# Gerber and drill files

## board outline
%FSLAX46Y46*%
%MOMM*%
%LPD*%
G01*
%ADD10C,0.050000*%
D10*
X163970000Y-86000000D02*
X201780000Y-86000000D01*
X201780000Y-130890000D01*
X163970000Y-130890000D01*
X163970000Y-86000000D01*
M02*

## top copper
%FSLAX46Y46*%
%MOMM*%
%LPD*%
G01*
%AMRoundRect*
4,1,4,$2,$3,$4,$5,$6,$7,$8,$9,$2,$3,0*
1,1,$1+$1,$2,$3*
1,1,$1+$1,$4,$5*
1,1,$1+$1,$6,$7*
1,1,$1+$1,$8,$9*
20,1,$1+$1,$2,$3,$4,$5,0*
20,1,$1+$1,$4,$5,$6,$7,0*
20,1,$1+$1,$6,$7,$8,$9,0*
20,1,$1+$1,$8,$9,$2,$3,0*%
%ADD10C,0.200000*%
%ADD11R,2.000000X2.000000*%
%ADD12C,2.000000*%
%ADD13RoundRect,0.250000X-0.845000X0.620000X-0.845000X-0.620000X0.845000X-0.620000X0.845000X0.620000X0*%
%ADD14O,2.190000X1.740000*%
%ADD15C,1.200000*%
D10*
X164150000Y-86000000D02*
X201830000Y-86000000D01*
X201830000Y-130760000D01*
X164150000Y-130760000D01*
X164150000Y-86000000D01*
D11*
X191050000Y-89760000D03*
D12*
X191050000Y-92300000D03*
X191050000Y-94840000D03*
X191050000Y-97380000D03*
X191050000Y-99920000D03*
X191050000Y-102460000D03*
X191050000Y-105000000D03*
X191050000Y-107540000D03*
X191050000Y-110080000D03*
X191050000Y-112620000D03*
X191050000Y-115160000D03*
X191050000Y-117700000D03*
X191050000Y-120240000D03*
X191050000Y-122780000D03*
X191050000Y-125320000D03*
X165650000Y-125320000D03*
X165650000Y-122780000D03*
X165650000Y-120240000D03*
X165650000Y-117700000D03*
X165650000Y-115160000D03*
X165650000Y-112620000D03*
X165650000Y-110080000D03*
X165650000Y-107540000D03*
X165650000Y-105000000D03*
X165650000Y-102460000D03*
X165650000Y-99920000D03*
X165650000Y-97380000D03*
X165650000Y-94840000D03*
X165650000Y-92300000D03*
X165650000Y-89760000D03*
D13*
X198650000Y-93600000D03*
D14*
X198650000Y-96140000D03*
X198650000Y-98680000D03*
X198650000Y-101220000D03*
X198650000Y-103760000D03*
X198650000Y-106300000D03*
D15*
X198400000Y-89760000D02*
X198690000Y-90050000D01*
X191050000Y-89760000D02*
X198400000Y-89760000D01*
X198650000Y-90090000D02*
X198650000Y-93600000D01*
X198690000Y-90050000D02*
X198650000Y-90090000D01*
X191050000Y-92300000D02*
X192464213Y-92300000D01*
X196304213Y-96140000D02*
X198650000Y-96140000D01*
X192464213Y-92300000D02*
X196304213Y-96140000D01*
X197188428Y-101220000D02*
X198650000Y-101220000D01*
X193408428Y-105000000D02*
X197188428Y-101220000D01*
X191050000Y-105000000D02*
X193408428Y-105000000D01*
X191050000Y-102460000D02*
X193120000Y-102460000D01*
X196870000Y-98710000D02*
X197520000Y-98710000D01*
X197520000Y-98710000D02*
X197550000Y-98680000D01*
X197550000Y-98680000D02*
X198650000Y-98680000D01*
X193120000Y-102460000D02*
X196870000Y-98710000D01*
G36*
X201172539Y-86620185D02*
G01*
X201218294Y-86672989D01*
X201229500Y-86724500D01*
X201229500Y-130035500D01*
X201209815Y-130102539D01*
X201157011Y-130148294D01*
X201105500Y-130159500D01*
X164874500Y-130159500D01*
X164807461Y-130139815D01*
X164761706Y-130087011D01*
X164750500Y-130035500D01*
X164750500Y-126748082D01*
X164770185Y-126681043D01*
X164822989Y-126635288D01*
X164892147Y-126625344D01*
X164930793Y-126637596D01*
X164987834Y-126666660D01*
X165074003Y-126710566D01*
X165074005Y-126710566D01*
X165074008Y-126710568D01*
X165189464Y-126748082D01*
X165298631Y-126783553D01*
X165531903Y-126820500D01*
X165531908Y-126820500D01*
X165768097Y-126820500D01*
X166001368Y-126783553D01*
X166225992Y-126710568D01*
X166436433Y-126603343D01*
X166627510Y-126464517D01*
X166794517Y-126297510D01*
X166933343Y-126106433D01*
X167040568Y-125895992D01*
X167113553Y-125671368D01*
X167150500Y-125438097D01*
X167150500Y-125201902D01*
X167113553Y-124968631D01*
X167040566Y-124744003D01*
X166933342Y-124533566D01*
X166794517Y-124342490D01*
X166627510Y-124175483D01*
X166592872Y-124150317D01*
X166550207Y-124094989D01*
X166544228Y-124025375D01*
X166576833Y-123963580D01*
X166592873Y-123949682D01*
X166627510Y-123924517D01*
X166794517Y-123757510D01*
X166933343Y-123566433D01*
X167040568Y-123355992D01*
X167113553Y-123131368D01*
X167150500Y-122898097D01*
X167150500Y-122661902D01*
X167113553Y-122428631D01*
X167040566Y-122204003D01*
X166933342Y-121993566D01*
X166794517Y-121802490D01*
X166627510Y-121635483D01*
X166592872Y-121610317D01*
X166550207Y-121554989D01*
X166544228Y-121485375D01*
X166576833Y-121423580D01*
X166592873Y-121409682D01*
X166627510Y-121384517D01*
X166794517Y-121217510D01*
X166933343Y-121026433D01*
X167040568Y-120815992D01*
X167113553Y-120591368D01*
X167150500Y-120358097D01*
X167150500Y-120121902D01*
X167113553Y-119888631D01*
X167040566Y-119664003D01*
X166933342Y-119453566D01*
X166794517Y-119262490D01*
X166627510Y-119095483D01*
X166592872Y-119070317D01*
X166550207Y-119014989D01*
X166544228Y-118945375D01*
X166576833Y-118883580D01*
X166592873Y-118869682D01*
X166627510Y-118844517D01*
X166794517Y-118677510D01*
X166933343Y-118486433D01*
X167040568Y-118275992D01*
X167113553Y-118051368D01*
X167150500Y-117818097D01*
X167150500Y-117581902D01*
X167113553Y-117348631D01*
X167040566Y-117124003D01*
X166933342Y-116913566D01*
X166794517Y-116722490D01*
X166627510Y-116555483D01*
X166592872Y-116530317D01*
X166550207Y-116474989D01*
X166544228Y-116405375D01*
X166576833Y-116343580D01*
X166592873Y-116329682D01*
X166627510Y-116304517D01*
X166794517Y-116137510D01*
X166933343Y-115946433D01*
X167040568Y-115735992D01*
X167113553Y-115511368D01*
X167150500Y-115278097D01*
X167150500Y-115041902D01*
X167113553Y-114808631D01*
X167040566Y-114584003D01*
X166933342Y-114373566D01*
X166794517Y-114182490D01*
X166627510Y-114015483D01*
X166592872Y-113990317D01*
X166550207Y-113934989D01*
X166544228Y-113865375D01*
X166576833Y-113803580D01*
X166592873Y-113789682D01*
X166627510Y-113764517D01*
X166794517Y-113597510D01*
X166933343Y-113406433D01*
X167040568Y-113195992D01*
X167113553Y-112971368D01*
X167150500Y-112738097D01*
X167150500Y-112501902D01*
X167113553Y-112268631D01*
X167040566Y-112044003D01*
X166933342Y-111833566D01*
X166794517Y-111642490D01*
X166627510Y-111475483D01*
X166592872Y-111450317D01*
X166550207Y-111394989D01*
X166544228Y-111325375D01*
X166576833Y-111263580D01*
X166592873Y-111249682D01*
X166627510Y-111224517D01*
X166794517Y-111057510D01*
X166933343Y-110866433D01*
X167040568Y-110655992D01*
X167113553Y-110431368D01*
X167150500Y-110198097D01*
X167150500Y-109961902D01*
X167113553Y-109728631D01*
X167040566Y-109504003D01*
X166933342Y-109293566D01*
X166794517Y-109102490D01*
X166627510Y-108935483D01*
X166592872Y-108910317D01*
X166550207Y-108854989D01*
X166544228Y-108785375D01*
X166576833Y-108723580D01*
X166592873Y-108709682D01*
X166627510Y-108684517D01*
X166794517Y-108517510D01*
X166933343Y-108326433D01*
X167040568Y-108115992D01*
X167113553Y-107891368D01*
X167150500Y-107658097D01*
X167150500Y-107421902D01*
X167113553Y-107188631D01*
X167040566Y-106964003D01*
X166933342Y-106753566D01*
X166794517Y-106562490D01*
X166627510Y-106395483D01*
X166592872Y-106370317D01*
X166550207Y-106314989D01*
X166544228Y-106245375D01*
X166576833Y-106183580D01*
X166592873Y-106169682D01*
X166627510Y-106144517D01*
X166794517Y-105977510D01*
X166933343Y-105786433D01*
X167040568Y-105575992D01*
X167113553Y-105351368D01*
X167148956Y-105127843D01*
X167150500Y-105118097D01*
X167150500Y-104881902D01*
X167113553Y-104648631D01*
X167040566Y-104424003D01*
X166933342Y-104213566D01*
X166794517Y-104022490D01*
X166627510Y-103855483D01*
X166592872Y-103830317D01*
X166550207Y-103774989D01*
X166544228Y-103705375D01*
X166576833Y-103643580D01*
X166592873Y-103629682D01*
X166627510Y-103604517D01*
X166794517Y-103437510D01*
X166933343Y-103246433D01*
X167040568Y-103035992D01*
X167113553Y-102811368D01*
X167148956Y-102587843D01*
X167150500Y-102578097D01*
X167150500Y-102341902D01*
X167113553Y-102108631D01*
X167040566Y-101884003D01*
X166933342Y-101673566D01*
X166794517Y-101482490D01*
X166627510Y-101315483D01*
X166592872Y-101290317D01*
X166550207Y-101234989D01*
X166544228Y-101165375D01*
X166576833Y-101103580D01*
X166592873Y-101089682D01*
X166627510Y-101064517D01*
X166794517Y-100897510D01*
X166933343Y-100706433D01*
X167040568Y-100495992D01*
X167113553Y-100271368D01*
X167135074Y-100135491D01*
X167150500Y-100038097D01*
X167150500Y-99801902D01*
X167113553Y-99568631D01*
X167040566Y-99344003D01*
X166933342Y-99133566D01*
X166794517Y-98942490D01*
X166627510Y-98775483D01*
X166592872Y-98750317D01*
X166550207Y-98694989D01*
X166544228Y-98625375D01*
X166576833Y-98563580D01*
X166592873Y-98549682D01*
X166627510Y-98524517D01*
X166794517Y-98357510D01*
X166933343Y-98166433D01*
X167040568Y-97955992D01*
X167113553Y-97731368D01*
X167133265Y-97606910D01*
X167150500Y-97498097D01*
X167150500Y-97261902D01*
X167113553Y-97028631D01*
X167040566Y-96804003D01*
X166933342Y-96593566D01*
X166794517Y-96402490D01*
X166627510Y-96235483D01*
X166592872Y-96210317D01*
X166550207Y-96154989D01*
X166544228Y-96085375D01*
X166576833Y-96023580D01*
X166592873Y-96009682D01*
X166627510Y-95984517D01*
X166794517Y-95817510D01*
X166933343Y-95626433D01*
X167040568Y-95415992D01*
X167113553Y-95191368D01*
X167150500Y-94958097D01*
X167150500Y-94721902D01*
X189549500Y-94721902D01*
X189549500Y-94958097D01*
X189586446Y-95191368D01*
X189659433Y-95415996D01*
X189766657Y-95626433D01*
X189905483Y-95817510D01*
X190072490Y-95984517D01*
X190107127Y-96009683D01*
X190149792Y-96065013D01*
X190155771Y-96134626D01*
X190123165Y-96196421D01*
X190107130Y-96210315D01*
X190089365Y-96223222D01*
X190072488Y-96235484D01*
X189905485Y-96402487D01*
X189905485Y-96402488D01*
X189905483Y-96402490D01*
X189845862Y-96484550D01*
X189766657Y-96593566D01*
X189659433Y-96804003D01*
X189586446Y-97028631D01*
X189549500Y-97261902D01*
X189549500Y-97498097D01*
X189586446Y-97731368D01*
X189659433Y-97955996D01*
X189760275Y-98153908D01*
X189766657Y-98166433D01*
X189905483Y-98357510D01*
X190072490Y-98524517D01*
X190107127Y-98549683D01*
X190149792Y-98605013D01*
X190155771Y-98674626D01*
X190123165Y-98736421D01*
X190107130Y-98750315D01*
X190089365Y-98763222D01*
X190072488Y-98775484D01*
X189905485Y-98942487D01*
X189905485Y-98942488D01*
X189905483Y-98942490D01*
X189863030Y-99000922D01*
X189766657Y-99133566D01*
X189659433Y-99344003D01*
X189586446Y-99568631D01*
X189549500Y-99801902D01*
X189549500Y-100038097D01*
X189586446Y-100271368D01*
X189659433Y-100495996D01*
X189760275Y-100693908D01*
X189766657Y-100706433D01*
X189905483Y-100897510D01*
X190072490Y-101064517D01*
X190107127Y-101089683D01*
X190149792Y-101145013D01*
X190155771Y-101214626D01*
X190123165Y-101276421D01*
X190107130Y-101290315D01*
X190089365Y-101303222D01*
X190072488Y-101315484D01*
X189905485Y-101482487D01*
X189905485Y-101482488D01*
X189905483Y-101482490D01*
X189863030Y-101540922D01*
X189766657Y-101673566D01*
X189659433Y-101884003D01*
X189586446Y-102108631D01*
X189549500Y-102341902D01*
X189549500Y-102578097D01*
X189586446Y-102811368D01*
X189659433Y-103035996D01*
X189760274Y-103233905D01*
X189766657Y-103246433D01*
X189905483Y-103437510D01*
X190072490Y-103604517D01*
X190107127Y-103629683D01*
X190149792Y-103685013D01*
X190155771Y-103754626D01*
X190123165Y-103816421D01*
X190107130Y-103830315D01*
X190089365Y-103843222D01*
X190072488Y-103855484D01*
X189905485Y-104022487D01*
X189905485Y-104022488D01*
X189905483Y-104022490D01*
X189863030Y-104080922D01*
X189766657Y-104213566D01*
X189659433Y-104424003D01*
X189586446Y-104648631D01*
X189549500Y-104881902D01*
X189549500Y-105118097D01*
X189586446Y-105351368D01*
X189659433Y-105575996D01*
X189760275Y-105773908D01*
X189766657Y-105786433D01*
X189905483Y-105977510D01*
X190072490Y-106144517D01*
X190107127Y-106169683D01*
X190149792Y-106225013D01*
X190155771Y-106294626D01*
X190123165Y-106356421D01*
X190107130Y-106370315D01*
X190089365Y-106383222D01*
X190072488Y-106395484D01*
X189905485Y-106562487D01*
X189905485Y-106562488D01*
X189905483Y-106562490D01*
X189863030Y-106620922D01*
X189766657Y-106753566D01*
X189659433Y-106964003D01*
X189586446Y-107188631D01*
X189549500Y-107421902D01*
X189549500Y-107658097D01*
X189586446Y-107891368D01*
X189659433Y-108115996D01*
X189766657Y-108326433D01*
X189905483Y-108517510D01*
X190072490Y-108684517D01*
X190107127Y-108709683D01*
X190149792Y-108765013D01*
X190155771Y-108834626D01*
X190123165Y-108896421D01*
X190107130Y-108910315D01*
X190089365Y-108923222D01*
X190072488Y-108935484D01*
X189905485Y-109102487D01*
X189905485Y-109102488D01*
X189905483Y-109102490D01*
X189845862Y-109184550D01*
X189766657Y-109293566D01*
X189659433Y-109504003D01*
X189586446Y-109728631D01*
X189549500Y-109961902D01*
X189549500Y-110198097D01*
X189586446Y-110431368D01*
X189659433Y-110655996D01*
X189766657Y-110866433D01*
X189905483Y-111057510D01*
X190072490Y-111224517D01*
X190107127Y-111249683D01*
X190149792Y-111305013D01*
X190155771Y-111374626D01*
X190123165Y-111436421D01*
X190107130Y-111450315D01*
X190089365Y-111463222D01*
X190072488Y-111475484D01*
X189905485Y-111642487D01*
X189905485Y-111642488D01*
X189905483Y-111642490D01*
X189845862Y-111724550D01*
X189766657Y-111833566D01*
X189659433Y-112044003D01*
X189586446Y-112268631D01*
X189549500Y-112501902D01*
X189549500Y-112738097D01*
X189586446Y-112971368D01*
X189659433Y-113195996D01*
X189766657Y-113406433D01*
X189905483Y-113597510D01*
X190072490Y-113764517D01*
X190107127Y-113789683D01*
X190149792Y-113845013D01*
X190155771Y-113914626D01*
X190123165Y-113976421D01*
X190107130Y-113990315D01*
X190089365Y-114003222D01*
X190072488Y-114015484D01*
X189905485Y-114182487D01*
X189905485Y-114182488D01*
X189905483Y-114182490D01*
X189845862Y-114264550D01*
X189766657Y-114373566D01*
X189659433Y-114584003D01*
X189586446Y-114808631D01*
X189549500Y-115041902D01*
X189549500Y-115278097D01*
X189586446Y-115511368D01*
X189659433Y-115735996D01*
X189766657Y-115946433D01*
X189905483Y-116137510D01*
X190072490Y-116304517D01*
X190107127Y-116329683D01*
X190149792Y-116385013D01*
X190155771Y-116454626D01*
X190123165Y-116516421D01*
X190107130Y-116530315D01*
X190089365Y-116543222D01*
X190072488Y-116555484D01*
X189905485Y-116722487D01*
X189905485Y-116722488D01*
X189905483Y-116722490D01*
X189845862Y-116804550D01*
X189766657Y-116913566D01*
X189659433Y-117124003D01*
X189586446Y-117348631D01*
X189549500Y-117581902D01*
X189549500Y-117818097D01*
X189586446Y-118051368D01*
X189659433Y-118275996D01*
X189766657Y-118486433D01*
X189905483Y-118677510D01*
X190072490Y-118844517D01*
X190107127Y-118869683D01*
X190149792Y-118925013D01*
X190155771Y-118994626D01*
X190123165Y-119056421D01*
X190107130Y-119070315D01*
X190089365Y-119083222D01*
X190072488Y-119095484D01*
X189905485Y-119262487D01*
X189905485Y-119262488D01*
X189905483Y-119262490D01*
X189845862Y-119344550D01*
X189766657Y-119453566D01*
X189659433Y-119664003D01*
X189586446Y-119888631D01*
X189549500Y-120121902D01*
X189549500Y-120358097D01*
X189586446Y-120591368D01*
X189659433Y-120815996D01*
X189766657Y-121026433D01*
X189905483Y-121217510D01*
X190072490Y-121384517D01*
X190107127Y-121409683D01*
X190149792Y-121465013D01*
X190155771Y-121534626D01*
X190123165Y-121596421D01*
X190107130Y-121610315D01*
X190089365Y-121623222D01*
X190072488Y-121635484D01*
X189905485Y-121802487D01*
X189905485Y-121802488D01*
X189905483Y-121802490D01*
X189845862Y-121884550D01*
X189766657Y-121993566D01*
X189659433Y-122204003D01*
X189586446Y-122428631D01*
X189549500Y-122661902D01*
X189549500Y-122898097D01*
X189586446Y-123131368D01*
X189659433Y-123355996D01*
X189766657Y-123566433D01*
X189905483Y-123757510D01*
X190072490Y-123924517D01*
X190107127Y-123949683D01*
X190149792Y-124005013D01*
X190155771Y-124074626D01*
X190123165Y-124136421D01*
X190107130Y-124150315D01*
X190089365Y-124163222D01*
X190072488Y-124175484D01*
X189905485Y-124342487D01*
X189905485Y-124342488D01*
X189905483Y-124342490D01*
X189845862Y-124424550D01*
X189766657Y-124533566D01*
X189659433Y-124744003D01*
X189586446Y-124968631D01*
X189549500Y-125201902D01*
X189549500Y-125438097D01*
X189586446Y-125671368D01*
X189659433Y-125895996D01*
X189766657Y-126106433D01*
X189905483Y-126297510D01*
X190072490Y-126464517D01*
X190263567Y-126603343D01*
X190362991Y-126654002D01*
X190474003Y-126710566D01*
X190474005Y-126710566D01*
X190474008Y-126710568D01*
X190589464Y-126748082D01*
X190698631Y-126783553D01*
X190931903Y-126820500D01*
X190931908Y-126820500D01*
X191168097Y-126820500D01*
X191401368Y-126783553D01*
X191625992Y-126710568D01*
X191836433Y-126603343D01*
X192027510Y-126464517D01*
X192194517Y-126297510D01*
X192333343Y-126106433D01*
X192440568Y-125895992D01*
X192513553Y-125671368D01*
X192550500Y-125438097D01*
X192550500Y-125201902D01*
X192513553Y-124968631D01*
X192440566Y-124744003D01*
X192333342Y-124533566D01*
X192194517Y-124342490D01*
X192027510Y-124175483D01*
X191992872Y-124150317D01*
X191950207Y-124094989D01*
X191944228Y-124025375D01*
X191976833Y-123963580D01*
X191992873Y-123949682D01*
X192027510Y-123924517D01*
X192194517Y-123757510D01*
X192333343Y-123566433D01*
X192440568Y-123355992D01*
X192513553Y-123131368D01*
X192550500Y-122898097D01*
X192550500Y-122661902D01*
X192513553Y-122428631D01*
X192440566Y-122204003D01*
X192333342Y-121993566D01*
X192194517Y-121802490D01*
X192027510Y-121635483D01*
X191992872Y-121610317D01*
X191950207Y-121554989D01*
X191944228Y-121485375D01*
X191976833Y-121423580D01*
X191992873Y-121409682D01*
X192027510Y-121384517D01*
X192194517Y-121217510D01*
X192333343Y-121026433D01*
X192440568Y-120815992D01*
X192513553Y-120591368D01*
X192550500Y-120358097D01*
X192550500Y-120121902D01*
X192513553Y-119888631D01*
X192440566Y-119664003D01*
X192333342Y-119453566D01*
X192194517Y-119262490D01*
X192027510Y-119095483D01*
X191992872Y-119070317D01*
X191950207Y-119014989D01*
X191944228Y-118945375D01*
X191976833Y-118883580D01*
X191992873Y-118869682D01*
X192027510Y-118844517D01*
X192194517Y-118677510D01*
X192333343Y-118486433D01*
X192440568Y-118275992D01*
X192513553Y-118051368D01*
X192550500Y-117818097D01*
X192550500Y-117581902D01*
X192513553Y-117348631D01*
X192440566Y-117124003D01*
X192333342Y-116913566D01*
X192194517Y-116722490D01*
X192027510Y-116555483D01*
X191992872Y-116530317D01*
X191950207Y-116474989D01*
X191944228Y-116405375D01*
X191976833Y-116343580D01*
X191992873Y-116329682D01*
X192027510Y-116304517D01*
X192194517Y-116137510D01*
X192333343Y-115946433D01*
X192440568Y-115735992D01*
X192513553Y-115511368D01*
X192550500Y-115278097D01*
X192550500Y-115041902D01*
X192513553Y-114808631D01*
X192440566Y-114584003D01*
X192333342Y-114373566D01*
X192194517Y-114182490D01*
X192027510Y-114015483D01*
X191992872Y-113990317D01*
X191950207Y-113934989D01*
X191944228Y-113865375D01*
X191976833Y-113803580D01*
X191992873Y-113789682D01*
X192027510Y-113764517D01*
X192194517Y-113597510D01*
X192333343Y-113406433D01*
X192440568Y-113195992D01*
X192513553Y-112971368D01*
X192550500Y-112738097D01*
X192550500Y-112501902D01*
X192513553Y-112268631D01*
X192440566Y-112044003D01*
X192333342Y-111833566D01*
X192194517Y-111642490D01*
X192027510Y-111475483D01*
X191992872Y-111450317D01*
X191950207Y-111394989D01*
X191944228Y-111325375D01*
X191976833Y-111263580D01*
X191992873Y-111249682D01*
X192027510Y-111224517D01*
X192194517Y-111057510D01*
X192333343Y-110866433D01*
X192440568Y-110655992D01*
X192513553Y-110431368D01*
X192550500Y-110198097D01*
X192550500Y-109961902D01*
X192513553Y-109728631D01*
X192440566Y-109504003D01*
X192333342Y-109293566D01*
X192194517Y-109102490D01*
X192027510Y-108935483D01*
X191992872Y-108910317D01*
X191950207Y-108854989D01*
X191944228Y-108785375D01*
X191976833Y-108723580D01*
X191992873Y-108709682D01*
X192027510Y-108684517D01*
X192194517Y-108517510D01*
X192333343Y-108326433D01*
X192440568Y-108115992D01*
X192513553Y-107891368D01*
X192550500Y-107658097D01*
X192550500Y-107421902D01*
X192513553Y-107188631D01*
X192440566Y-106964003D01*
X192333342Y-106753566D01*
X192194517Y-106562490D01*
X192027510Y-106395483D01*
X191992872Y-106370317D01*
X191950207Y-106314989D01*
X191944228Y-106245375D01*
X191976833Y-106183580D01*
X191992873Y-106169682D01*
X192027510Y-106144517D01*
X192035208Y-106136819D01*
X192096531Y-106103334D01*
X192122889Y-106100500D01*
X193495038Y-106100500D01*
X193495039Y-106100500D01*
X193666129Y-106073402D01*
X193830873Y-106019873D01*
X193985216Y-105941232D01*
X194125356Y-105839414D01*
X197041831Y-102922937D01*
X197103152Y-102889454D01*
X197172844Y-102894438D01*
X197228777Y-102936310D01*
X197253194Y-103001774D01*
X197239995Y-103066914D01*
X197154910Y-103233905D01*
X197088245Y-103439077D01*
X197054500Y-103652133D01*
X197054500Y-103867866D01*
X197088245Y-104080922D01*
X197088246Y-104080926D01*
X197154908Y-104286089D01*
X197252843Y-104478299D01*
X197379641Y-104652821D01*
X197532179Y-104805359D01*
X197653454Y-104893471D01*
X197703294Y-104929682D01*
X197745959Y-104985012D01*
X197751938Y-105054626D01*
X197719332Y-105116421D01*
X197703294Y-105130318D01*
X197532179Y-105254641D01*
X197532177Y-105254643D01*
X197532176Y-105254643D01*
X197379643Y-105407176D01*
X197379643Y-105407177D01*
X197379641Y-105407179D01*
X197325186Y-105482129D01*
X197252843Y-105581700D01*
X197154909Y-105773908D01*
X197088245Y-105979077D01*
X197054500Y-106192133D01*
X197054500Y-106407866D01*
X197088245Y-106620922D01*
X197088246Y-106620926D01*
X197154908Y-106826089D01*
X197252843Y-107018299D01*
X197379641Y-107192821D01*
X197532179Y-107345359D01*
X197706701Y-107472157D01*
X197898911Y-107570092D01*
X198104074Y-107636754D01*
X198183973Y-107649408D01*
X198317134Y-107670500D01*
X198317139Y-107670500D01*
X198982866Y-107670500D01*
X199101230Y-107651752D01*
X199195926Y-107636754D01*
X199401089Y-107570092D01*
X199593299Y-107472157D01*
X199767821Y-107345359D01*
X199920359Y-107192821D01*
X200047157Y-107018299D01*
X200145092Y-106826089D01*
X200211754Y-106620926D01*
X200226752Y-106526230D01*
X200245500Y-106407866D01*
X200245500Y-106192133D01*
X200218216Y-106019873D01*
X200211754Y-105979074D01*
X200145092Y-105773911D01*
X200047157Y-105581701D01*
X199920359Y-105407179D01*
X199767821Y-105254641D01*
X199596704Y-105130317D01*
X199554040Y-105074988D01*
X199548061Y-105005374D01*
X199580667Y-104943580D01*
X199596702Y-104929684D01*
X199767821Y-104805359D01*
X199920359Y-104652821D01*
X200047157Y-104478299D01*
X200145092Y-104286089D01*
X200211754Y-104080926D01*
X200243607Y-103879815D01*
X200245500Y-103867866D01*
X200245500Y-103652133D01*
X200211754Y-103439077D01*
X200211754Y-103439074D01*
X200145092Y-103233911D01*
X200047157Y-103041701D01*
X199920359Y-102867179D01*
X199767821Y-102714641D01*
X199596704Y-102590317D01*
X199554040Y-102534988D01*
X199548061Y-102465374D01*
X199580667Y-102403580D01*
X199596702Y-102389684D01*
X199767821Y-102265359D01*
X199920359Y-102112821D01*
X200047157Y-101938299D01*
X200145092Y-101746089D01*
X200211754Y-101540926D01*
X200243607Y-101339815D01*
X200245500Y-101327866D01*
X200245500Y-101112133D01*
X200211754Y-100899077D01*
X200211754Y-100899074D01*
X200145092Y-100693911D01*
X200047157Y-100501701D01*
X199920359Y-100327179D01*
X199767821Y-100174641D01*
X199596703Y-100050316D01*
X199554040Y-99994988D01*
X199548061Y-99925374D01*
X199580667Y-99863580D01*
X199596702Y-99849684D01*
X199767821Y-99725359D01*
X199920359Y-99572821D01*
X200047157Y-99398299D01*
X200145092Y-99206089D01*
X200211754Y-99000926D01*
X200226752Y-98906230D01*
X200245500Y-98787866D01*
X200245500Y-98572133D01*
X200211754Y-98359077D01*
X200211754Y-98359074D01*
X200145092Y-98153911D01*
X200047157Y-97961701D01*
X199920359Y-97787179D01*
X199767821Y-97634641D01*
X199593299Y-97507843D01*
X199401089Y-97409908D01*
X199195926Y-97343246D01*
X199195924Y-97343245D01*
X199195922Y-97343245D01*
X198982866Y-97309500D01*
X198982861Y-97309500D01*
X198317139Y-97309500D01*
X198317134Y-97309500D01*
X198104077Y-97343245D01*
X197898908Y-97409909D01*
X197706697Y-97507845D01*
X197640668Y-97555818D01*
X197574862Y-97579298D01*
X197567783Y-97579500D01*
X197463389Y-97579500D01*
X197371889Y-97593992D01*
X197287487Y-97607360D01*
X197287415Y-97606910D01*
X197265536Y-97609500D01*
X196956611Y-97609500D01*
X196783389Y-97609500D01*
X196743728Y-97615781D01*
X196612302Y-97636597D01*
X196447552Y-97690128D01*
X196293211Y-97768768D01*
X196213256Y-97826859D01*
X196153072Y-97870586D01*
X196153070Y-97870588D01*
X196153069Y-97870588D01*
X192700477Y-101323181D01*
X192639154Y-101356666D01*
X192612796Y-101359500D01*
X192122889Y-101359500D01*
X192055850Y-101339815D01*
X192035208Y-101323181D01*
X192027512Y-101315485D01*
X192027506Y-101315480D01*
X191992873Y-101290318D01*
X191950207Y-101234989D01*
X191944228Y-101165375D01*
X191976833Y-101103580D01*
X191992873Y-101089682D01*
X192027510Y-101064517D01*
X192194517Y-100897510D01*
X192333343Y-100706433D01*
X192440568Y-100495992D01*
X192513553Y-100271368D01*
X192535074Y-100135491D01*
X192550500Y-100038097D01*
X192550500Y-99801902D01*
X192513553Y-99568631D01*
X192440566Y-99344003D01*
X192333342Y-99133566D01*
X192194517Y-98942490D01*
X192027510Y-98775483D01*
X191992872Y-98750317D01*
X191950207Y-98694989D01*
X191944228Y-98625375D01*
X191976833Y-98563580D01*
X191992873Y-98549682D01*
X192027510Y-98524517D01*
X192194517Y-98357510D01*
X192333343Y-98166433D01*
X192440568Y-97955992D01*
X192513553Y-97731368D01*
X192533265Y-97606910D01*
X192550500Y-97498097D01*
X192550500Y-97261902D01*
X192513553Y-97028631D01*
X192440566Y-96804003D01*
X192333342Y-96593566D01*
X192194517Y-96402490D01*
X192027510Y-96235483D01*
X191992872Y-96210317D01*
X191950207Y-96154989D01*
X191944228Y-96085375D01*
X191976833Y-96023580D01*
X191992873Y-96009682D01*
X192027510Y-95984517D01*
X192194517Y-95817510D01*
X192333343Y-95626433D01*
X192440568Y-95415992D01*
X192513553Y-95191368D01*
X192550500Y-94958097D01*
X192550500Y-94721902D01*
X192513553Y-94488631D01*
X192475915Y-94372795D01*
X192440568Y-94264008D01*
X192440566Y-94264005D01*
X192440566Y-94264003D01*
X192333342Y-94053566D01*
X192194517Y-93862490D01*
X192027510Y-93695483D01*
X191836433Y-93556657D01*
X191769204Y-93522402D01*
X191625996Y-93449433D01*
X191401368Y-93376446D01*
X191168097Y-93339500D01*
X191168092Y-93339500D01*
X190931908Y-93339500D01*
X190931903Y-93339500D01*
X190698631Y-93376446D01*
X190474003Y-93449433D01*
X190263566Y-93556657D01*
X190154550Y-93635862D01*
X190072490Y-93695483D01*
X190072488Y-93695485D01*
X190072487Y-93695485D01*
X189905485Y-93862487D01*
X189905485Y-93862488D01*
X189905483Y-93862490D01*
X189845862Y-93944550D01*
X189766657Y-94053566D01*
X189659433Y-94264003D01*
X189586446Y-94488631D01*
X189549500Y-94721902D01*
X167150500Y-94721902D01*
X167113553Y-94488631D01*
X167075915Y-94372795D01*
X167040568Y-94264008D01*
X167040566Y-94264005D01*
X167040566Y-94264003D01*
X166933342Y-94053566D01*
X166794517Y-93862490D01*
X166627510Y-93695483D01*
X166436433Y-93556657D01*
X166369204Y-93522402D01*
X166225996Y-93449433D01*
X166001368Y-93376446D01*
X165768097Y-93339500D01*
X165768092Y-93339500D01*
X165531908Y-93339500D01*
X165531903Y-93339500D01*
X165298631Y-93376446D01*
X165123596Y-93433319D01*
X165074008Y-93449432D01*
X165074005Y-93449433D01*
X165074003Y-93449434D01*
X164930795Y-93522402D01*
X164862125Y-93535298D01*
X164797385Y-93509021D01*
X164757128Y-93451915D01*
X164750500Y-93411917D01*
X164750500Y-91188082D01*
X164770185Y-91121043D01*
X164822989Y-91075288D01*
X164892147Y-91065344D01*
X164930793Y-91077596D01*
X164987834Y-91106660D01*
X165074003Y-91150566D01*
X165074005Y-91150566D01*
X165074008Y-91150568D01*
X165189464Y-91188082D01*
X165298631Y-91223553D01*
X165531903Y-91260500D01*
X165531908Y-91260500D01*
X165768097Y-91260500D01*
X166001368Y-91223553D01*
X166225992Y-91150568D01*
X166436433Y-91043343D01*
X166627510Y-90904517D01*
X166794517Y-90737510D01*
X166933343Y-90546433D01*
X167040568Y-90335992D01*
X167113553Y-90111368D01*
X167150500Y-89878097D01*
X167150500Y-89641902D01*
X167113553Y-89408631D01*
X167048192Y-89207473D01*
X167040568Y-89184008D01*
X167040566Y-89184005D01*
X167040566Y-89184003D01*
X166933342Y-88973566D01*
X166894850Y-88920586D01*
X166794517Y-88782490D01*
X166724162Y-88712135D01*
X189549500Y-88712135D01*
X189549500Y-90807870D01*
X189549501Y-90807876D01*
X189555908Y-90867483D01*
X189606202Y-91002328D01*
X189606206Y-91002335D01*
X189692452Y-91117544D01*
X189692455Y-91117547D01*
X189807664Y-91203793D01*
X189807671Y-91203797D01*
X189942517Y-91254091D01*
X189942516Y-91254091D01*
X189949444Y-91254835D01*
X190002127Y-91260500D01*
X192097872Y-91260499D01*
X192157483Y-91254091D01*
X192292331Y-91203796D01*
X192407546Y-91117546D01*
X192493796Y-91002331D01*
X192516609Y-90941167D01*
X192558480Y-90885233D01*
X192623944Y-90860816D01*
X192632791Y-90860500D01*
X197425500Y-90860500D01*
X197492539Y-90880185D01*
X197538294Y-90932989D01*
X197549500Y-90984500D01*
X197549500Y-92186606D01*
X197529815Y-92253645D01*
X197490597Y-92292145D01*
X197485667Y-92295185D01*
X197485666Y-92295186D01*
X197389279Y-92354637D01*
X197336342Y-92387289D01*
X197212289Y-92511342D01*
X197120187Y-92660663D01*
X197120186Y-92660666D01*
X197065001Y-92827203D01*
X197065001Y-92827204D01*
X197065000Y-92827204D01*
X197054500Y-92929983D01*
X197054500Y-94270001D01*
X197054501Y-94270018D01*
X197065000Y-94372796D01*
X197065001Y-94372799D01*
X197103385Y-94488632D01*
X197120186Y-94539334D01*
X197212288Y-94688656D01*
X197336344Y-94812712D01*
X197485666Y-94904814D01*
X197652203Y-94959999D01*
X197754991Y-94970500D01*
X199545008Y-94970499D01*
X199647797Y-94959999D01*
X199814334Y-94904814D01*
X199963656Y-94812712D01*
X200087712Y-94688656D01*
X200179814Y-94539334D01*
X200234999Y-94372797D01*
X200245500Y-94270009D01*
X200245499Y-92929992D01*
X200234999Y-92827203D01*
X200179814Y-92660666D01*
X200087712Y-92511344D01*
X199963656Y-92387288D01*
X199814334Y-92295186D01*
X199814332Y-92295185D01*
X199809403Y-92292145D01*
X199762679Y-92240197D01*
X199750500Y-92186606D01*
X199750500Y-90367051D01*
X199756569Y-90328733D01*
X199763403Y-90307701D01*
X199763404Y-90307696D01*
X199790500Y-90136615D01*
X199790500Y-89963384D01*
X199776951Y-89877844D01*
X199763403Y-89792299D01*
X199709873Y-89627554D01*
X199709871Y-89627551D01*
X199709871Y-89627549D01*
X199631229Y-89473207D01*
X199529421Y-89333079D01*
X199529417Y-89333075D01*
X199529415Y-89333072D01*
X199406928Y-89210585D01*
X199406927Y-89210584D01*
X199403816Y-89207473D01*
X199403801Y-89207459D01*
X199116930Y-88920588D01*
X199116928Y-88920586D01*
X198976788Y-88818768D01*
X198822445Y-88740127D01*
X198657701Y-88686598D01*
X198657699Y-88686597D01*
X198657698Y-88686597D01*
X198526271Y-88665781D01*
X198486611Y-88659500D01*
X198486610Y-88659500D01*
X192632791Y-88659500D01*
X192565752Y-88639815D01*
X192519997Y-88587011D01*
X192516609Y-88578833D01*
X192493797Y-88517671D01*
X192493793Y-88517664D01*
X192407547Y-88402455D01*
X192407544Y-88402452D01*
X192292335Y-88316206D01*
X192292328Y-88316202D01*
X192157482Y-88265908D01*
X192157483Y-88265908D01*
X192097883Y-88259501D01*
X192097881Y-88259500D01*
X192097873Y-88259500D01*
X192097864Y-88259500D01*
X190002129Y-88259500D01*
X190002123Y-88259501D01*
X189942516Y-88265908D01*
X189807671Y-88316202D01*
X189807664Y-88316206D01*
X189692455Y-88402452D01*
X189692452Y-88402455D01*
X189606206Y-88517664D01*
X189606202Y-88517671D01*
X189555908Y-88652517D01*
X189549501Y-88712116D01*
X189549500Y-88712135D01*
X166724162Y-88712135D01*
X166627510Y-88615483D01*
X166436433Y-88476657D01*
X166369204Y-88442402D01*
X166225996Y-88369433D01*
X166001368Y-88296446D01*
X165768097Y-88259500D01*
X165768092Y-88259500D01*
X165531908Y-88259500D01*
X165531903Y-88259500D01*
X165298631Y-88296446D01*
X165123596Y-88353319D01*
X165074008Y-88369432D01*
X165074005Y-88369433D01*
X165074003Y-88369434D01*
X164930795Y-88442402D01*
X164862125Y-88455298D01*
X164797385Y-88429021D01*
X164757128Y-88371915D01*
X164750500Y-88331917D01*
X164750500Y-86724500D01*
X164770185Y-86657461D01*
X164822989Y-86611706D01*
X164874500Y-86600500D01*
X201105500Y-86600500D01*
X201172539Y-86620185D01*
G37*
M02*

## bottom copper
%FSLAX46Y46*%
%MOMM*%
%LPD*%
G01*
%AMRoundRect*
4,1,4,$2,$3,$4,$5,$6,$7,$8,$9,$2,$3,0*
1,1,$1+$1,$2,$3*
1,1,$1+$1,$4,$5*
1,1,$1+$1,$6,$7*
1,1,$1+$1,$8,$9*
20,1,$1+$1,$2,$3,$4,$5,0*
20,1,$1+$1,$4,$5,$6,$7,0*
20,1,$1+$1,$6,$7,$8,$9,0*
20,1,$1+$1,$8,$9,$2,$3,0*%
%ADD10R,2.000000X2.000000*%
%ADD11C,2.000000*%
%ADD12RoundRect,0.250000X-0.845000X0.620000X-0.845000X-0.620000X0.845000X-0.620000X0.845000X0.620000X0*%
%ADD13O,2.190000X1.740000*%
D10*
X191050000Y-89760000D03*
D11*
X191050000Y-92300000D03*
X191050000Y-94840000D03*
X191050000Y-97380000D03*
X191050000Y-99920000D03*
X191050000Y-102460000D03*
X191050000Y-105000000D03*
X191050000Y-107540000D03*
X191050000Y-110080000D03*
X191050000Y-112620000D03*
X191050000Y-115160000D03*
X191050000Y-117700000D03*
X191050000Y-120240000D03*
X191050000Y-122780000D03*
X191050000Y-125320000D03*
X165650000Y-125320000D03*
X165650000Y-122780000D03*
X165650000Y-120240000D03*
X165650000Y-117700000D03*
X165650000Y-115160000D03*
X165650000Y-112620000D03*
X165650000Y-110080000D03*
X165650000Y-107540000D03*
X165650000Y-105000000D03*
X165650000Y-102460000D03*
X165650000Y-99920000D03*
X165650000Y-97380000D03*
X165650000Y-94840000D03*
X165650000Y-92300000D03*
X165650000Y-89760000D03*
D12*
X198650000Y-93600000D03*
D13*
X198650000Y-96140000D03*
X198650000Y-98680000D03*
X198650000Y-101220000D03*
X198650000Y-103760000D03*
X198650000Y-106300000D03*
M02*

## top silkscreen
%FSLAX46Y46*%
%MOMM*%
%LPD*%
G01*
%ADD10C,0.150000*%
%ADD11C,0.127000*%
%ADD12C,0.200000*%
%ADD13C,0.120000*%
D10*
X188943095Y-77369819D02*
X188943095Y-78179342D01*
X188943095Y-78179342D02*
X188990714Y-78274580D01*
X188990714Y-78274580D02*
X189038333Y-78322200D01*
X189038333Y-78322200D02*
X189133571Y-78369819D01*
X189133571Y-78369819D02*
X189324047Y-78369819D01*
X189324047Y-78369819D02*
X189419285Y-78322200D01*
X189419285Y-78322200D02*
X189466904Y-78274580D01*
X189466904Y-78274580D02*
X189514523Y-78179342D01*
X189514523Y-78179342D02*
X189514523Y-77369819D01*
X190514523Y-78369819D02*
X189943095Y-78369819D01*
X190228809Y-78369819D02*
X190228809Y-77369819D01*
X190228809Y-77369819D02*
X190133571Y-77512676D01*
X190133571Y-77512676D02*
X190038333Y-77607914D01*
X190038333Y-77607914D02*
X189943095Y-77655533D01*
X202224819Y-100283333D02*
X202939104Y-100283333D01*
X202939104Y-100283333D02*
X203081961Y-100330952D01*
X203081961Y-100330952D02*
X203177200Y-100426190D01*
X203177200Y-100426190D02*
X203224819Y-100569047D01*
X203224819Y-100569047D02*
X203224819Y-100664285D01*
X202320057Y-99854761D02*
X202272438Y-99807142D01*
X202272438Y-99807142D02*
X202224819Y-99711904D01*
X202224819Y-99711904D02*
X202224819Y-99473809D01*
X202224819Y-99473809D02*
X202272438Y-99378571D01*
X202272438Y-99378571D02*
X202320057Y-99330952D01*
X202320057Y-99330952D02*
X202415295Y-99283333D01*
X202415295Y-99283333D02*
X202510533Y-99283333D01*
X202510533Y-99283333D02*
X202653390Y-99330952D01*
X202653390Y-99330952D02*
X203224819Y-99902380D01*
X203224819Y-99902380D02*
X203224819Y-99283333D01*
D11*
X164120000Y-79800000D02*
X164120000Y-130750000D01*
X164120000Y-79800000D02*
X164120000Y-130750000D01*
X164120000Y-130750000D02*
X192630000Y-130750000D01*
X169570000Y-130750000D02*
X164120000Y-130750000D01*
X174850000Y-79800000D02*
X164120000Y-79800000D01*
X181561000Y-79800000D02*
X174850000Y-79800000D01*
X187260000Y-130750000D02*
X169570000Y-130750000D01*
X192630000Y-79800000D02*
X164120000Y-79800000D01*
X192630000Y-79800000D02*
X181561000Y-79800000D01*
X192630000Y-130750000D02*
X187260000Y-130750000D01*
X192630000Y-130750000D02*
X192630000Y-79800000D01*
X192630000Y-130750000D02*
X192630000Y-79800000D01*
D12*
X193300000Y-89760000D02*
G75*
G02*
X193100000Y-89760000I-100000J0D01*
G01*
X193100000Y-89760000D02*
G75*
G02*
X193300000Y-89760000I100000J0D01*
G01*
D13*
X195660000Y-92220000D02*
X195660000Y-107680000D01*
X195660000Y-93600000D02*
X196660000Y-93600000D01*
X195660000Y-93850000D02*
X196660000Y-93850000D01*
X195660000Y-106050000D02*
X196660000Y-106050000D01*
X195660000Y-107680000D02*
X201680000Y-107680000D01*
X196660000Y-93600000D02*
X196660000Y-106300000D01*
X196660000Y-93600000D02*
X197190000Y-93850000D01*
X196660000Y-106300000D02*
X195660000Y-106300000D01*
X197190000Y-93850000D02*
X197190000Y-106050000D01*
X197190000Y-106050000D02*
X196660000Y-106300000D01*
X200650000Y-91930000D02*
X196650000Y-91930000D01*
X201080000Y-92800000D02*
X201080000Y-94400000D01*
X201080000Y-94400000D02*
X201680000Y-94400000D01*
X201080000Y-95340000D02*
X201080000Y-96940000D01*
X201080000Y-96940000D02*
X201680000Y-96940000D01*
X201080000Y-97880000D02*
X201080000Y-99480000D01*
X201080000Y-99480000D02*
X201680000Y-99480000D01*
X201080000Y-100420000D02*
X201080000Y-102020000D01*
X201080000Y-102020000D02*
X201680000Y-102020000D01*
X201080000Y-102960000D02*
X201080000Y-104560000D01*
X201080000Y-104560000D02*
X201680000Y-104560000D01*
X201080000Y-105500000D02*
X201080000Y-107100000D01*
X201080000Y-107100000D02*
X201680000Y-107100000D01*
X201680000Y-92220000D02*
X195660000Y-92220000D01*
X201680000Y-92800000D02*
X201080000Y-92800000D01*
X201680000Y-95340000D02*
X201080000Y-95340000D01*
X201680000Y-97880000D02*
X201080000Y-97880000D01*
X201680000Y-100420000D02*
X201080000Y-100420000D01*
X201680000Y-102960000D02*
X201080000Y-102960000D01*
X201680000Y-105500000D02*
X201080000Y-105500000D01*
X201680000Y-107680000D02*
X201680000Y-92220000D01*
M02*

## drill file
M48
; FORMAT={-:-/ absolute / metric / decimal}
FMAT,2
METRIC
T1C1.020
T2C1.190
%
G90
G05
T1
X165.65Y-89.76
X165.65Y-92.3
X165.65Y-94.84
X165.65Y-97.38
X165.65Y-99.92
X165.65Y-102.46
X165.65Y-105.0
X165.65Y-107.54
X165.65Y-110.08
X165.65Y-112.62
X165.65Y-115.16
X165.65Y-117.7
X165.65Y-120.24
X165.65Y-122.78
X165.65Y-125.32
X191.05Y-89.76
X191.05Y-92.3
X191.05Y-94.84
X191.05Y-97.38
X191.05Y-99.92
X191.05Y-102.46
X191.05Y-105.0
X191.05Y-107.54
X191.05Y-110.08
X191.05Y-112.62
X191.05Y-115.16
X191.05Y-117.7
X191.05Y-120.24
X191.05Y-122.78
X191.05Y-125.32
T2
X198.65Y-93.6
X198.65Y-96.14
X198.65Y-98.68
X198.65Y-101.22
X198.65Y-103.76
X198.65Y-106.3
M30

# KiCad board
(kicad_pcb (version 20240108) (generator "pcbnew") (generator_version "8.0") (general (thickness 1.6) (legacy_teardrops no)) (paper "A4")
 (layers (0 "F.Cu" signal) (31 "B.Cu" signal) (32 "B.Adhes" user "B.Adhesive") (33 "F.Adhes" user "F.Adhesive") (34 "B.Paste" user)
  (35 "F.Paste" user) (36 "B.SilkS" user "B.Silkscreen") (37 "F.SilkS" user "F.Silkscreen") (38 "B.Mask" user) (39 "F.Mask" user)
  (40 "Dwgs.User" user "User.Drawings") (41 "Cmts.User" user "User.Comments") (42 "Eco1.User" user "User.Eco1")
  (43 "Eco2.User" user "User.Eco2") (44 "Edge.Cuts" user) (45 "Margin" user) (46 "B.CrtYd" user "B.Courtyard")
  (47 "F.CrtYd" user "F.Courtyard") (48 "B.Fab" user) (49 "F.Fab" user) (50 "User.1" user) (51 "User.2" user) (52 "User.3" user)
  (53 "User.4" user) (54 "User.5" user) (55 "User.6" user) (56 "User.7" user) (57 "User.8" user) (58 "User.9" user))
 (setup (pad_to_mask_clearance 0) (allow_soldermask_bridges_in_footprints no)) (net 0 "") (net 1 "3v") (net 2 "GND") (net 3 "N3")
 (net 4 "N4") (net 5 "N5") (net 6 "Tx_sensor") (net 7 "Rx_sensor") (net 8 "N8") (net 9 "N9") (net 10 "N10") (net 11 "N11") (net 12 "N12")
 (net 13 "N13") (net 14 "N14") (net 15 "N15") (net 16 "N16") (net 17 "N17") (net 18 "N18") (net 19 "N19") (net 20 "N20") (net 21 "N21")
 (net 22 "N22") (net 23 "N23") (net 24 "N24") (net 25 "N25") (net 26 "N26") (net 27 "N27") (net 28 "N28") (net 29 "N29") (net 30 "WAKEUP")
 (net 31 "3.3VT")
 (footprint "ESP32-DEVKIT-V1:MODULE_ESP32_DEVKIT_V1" (layer "F.Cu") (at 178.35 105.275)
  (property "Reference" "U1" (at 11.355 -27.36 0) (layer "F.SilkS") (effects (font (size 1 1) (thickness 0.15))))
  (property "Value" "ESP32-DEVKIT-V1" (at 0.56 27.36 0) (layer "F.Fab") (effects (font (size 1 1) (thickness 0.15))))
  (fp_line (start -14.23 -25.475) (end -14.23 25.475) (stroke (width 0.127) (type solid)) (layer "F.SilkS"))
  (fp_line (start -14.23 -25.475) (end -14.23 25.475) (stroke (width 0.127) (type solid)) (layer "F.SilkS"))
  (fp_line (start -14.23 25.475) (end 14.28 25.475) (stroke (width 0.127) (type solid)) (layer "F.SilkS"))
  (fp_line (start -8.78 25.475) (end -14.23 25.475) (stroke (width 0.127) (type solid)) (layer "F.SilkS"))
  (fp_line (start -3.5 -25.475) (end -14.23 -25.475) (stroke (width 0.127) (type solid)) (layer "F.SilkS"))
  (fp_line (start 3.211 -25.475) (end -3.5 -25.475) (stroke (width 0.127) (type solid)) (layer "F.SilkS"))
  (fp_line (start 8.91 25.475) (end -8.78 25.475) (stroke (width 0.127) (type solid)) (layer "F.SilkS"))
  (fp_line (start 14.28 -25.475) (end -14.23 -25.475) (stroke (width 0.127) (type solid)) (layer "F.SilkS"))
  (fp_line (start 14.28 -25.475) (end 3.211 -25.475) (stroke (width 0.127) (type solid)) (layer "F.SilkS"))
  (fp_line (start 14.28 25.475) (end 8.91 25.475) (stroke (width 0.127) (type solid)) (layer "F.SilkS"))
  (fp_line (start 14.28 25.475) (end 14.28 -25.475) (stroke (width 0.127) (type solid)) (layer "F.SilkS"))
  (fp_line (start 14.28 25.475) (end 14.28 -25.475) (stroke (width 0.127) (type solid)) (layer "F.SilkS"))
  (fp_circle (center 14.85 -15.515) (end 14.75 -15.515) (stroke (width 0.2) (type solid)) (fill none) (layer "F.SilkS"))
  (pad "1" thru_hole rect (at 12.7 -15.515) (size 2 2) (drill 1.02) (layers "*.Cu" "*.Mask") (remove_unused_layers no) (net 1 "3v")
   (solder_mask_margin 0.102))
  (pad "2" thru_hole circle (at 12.7 -12.975) (size 2 2) (drill 1.02) (layers "*.Cu" "*.Mask") (remove_unused_layers no) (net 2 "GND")
   (solder_mask_margin 0.102))
  (pad "3" thru_hole circle (at 12.7 -10.435) (size 2 2) (drill 1.02) (layers "*.Cu" "*.Mask") (remove_unused_layers no) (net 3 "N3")
   (solder_mask_margin 0.102))
  (pad "4" thru_hole circle (at 12.7 -7.895) (size 2 2) (drill 1.02) (layers "*.Cu" "*.Mask") (remove_unused_layers no) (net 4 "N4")
   (solder_mask_margin 0.102))
  (pad "5" thru_hole circle (at 12.7 -5.355) (size 2 2) (drill 1.02) (layers "*.Cu" "*.Mask") (remove_unused_layers no) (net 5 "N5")
   (solder_mask_margin 0.102))
  (pad "6" thru_hole circle (at 12.7 -2.815) (size 2 2) (drill 1.02) (layers "*.Cu" "*.Mask") (remove_unused_layers no) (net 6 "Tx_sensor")
   (solder_mask_margin 0.102))
  (pad "7" thru_hole circle (at 12.7 -0.275) (size 2 2) (drill 1.02) (layers "*.Cu" "*.Mask") (remove_unused_layers no) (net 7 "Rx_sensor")
   (solder_mask_margin 0.102))
  (pad "8" thru_hole circle (at 12.7 2.265) (size 2 2) (drill 1.02) (layers "*.Cu" "*.Mask") (remove_unused_layers no) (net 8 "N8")
   (solder_mask_margin 0.102))
  (pad "9" thru_hole circle (at 12.7 4.805) (size 2 2) (drill 1.02) (layers "*.Cu" "*.Mask") (remove_unused_layers no) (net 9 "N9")
   (solder_mask_margin 0.102))
  (pad "10" thru_hole circle (at 12.7 7.345) (size 2 2) (drill 1.02) (layers "*.Cu" "*.Mask") (remove_unused_layers no) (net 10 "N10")
   (solder_mask_margin 0.102))
  (pad "11" thru_hole circle (at 12.7 9.885) (size 2 2) (drill 1.02) (layers "*.Cu" "*.Mask") (remove_unused_layers no) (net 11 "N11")
   (solder_mask_margin 0.102))
  (pad "12" thru_hole circle (at 12.7 12.425) (size 2 2) (drill 1.02) (layers "*.Cu" "*.Mask") (remove_unused_layers no) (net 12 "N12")
   (solder_mask_margin 0.102))
  (pad "13" thru_hole circle (at 12.7 14.965) (size 2 2) (drill 1.02) (layers "*.Cu" "*.Mask") (remove_unused_layers no) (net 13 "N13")
   (solder_mask_margin 0.102))
  (pad "14" thru_hole circle (at 12.7 17.505) (size 2 2) (drill 1.02) (layers "*.Cu" "*.Mask") (remove_unused_layers no) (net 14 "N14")
   (solder_mask_margin 0.102))
  (pad "15" thru_hole circle (at 12.7 20.045) (size 2 2) (drill 1.02) (layers "*.Cu" "*.Mask") (remove_unused_layers no) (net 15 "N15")
   (solder_mask_margin 0.102))
  (pad "16" thru_hole circle (at -12.7 20.045) (size 2 2) (drill 1.02) (layers "*.Cu" "*.Mask") (remove_unused_layers no) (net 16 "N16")
   (solder_mask_margin 0.102))
  (pad "17" thru_hole circle (at -12.7 17.505) (size 2 2) (drill 1.02) (layers "*.Cu" "*.Mask") (remove_unused_layers no) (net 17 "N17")
   (solder_mask_margin 0.102))
  (pad "18" thru_hole circle (at -12.7 14.965) (size 2 2) (drill 1.02) (layers "*.Cu" "*.Mask") (remove_unused_layers no) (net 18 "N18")
   (solder_mask_margin 0.102))
  (pad "19" thru_hole circle (at -12.7 12.425) (size 2 2) (drill 1.02) (layers "*.Cu" "*.Mask") (remove_unused_layers no) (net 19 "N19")
   (solder_mask_margin 0.102))
  (pad "20" thru_hole circle (at -12.7 9.885) (size 2 2) (drill 1.02) (layers "*.Cu" "*.Mask") (remove_unused_layers no) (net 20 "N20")
   (solder_mask_margin 0.102))
  (pad "21" thru_hole circle (at -12.7 7.345) (size 2 2) (drill 1.02) (layers "*.Cu" "*.Mask") (remove_unused_layers no) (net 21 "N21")
   (solder_mask_margin 0.102))
  (pad "22" thru_hole circle (at -12.7 4.805) (size 2 2) (drill 1.02) (layers "*.Cu" "*.Mask") (remove_unused_layers no) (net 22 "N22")
   (solder_mask_margin 0.102))
  (pad "23" thru_hole circle (at -12.7 2.265) (size 2 2) (drill 1.02) (layers "*.Cu" "*.Mask") (remove_unused_layers no) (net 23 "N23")
   (solder_mask_margin 0.102))
  (pad "24" thru_hole circle (at -12.7 -0.275) (size 2 2) (drill 1.02) (layers "*.Cu" "*.Mask") (remove_unused_layers no) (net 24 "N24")
   (solder_mask_margin 0.102))
  (pad "25" thru_hole circle (at -12.7 -2.815) (size 2 2) (drill 1.02) (layers "*.Cu" "*.Mask") (remove_unused_layers no) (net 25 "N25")
   (solder_mask_margin 0.102))
  (pad "26" thru_hole circle (at -12.7 -5.355) (size 2 2) (drill 1.02) (layers "*.Cu" "*.Mask") (remove_unused_layers no) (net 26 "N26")
   (solder_mask_margin 0.102))
  (pad "27" thru_hole circle (at -12.7 -7.895) (size 2 2) (drill 1.02) (layers "*.Cu" "*.Mask") (remove_unused_layers no) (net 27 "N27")
   (solder_mask_margin 0.102))
  (pad "28" thru_hole circle (at -12.7 -10.435) (size 2 2) (drill 1.02) (layers "*.Cu" "*.Mask") (remove_unused_layers no) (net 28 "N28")
   (solder_mask_margin 0.102))
  (pad "29" thru_hole circle (at -12.7 -12.975) (size 2 2) (drill 1.02) (layers "*.Cu" "*.Mask") (remove_unused_layers no) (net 2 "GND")
   (solder_mask_margin 0.102))
  (pad "30" thru_hole circle (at -12.7 -15.515) (size 2 2) (drill 1.02) (layers "*.Cu" "*.Mask") (remove_unused_layers no) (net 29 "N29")
   (solder_mask_margin 0.102)))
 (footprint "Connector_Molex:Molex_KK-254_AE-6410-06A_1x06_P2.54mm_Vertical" (layer "F.Cu") (at 198.65 93.6 -90)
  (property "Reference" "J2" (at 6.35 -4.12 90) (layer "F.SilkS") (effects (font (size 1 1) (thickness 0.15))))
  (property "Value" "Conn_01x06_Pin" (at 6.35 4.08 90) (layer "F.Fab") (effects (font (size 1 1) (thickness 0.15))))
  (fp_line (start -1.38 2.99) (end 14.08 2.99) (stroke (width 0.12) (type solid)) (layer "F.SilkS"))
  (fp_line (start 0 2.99) (end 0 1.99) (stroke (width 0.12) (type solid)) (layer "F.SilkS"))
  (fp_line (start 0.25 2.99) (end 0.25 1.99) (stroke (width 0.12) (type solid)) (layer "F.SilkS"))
  (fp_line (start 12.45 2.99) (end 12.45 1.99) (stroke (width 0.12) (type solid)) (layer "F.SilkS"))
  (fp_line (start 14.08 2.99) (end 14.08 -3.03) (stroke (width 0.12) (type solid)) (layer "F.SilkS"))
  (fp_line (start 0 1.99) (end 12.7 1.99) (stroke (width 0.12) (type solid)) (layer "F.SilkS"))
  (fp_line (start 0 1.99) (end 0.25 1.46) (stroke (width 0.12) (type solid)) (layer "F.SilkS"))
  (fp_line (start 12.7 1.99) (end 12.7 2.99) (stroke (width 0.12) (type solid)) (layer "F.SilkS"))
  (fp_line (start 0.25 1.46) (end 12.45 1.46) (stroke (width 0.12) (type solid)) (layer "F.SilkS"))
  (fp_line (start 12.45 1.46) (end 12.7 1.99) (stroke (width 0.12) (type solid)) (layer "F.SilkS"))
  (fp_line (start -1.67 -2) (end -1.67 2) (stroke (width 0.12) (type solid)) (layer "F.SilkS"))
  (fp_line (start -0.8 -2.43) (end 0.8 -2.43) (stroke (width 0.12) (type solid)) (layer "F.SilkS"))
  (fp_line (start 0.8 -2.43) (end 0.8 -3.03) (stroke (width 0.12) (type solid)) (layer "F.SilkS"))
  (fp_line (start 1.74 -2.43) (end 3.34 -2.43) (stroke (width 0.12) (type solid)) (layer "F.SilkS"))
  (fp_line (start 3.34 -2.43) (end 3.34 -3.03) (stroke (width 0.12) (type solid)) (layer "F.SilkS"))
  (fp_line (start 4.28 -2.43) (end 5.88 -2.43) (stroke (width 0.12) (type solid)) (layer "F.SilkS"))
  (fp_line (start 5.88 -2.43) (end 5.88 -3.03) (stroke (width 0.12) (type solid)) (layer "F.SilkS"))
  (fp_line (start 6.82 -2.43) (end 8.42 -2.43) (stroke (width 0.12) (type solid)) (layer "F.SilkS"))
  (fp_line (start 8.42 -2.43) (end 8.42 -3.03) (stroke (width 0.12) (type solid)) (layer "F.SilkS"))
  (fp_line (start 9.36 -2.43) (end 10.96 -2.43) (stroke (width 0.12) (type solid)) (layer "F.SilkS"))
  (fp_line (start 10.96 -2.43) (end 10.96 -3.03) (stroke (width 0.12) (type solid)) (layer "F.SilkS"))
  (fp_line (start 11.9 -2.43) (end 13.5 -2.43) (stroke (width 0.12) (type solid)) (layer "F.SilkS"))
  (fp_line (start 13.5 -2.43) (end 13.5 -3.03) (stroke (width 0.12) (type solid)) (layer "F.SilkS"))
  (fp_line (start -1.38 -3.03) (end -1.38 2.99) (stroke (width 0.12) (type solid)) (layer "F.SilkS"))
  (fp_line (start -0.8 -3.03) (end -0.8 -2.43) (stroke (width 0.12) (type solid)) (layer "F.SilkS"))
  (fp_line (start 1.74 -3.03) (end 1.74 -2.43) (stroke (width 0.12) (type solid)) (layer "F.SilkS"))
  (fp_line (start 4.28 -3.03) (end 4.28 -2.43) (stroke (width 0.12) (type solid)) (layer "F.SilkS"))
  (fp_line (start 6.82 -3.03) (end 6.82 -2.43) (stroke (width 0.12) (type solid)) (layer "F.SilkS"))
  (fp_line (start 9.36 -3.03) (end 9.36 -2.43) (stroke (width 0.12) (type solid)) (layer "F.SilkS"))
  (fp_line (start 11.9 -3.03) (end 11.9 -2.43) (stroke (width 0.12) (type solid)) (layer "F.SilkS"))
  (fp_line (start 14.08 -3.03) (end -1.38 -3.03) (stroke (width 0.12) (type solid)) (layer "F.SilkS"))
  (pad "1" thru_hole roundrect (at 0 0 270) (size 1.74 2.19) (drill 1.19) (layers "*.Cu" "*.Mask") (remove_unused_layers no)
   (roundrect_rratio 0.143678) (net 1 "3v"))
  (pad "2" thru_hole oval (at 2.54 0 270) (size 1.74 2.19) (drill 1.19) (layers "*.Cu" "*.Mask") (remove_unused_layers no) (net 2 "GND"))
  (pad "3" thru_hole oval (at 5.08 0 270) (size 1.74 2.19) (drill 1.19) (layers "*.Cu" "*.Mask") (remove_unused_layers no)
   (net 6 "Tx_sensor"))
  (pad "4" thru_hole oval (at 7.62 0 270) (size 1.74 2.19) (drill 1.19) (layers "*.Cu" "*.Mask") (remove_unused_layers no)
   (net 7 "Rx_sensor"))
  (pad "5" thru_hole oval (at 10.16 0 270) (size 1.74 2.19) (drill 1.19) (layers "*.Cu" "*.Mask") (remove_unused_layers no)
   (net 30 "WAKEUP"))
  (pad "6" thru_hole oval (at 12.7 0 270) (size 1.74 2.19) (drill 1.19) (layers "*.Cu" "*.Mask") (remove_unused_layers no) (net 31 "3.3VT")))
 (gr_rect (start 164.15 86) (end 201.83 130.76) (stroke (width 0.2) (type default)) (fill none) (layer "F.Cu"))
 (gr_rect (start 163.97 86) (end 201.78 130.89) (stroke (width 0.05) (type default)) (fill none) (layer "Edge.Cuts"))
 (segment (start 198.4 89.76) (end 198.69 90.05) (width 1.2) (layer "F.Cu") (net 1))
 (segment (start 191.05 89.76) (end 198.4 89.76) (width 1.2) (layer "F.Cu") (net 1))
 (segment (start 198.65 90.09) (end 198.65 93.6) (width 1.2) (layer "F.Cu") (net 1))
 (segment (start 198.69 90.05) (end 198.65 90.09) (width 1.2) (layer "F.Cu") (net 1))
 (segment (start 191.05 92.3) (end 192.464213 92.3) (width 1.2) (layer "F.Cu") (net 2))
 (segment (start 196.304213 96.14) (end 198.65 96.14) (width 1.2) (layer "F.Cu") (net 2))
 (segment (start 192.464213 92.3) (end 196.304213 96.14) (width 1.2) (layer "F.Cu") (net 2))
 (segment (start 197.188428 101.22) (end 198.65 101.22) (width 1.2) (layer "F.Cu") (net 7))
 (segment (start 193.408428 105) (end 197.188428 101.22) (width 1.2) (layer "F.Cu") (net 7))
 (segment (start 191.05 105) (end 193.408428 105) (width 1.2) (layer "F.Cu") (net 7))
 (segment (start 191.05 102.46) (end 193.12 102.46) (width 1.2) (layer "F.Cu") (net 6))
 (segment (start 196.87 98.71) (end 197.52 98.71) (width 1.2) (layer "F.Cu") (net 6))
 (segment (start 197.52 98.71) (end 197.55 98.68) (width 1.2) (layer "F.Cu") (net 6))
 (segment (start 197.55 98.68) (end 198.65 98.68) (width 1.2) (layer "F.Cu") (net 6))
 (segment (start 193.12 102.46) (end 196.87 98.71) (width 1.2) (layer "F.Cu") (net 6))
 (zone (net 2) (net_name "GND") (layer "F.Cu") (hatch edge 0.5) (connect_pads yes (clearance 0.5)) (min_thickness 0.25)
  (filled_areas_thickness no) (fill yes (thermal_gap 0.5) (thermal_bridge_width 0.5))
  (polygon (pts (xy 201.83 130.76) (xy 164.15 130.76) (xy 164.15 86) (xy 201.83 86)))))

